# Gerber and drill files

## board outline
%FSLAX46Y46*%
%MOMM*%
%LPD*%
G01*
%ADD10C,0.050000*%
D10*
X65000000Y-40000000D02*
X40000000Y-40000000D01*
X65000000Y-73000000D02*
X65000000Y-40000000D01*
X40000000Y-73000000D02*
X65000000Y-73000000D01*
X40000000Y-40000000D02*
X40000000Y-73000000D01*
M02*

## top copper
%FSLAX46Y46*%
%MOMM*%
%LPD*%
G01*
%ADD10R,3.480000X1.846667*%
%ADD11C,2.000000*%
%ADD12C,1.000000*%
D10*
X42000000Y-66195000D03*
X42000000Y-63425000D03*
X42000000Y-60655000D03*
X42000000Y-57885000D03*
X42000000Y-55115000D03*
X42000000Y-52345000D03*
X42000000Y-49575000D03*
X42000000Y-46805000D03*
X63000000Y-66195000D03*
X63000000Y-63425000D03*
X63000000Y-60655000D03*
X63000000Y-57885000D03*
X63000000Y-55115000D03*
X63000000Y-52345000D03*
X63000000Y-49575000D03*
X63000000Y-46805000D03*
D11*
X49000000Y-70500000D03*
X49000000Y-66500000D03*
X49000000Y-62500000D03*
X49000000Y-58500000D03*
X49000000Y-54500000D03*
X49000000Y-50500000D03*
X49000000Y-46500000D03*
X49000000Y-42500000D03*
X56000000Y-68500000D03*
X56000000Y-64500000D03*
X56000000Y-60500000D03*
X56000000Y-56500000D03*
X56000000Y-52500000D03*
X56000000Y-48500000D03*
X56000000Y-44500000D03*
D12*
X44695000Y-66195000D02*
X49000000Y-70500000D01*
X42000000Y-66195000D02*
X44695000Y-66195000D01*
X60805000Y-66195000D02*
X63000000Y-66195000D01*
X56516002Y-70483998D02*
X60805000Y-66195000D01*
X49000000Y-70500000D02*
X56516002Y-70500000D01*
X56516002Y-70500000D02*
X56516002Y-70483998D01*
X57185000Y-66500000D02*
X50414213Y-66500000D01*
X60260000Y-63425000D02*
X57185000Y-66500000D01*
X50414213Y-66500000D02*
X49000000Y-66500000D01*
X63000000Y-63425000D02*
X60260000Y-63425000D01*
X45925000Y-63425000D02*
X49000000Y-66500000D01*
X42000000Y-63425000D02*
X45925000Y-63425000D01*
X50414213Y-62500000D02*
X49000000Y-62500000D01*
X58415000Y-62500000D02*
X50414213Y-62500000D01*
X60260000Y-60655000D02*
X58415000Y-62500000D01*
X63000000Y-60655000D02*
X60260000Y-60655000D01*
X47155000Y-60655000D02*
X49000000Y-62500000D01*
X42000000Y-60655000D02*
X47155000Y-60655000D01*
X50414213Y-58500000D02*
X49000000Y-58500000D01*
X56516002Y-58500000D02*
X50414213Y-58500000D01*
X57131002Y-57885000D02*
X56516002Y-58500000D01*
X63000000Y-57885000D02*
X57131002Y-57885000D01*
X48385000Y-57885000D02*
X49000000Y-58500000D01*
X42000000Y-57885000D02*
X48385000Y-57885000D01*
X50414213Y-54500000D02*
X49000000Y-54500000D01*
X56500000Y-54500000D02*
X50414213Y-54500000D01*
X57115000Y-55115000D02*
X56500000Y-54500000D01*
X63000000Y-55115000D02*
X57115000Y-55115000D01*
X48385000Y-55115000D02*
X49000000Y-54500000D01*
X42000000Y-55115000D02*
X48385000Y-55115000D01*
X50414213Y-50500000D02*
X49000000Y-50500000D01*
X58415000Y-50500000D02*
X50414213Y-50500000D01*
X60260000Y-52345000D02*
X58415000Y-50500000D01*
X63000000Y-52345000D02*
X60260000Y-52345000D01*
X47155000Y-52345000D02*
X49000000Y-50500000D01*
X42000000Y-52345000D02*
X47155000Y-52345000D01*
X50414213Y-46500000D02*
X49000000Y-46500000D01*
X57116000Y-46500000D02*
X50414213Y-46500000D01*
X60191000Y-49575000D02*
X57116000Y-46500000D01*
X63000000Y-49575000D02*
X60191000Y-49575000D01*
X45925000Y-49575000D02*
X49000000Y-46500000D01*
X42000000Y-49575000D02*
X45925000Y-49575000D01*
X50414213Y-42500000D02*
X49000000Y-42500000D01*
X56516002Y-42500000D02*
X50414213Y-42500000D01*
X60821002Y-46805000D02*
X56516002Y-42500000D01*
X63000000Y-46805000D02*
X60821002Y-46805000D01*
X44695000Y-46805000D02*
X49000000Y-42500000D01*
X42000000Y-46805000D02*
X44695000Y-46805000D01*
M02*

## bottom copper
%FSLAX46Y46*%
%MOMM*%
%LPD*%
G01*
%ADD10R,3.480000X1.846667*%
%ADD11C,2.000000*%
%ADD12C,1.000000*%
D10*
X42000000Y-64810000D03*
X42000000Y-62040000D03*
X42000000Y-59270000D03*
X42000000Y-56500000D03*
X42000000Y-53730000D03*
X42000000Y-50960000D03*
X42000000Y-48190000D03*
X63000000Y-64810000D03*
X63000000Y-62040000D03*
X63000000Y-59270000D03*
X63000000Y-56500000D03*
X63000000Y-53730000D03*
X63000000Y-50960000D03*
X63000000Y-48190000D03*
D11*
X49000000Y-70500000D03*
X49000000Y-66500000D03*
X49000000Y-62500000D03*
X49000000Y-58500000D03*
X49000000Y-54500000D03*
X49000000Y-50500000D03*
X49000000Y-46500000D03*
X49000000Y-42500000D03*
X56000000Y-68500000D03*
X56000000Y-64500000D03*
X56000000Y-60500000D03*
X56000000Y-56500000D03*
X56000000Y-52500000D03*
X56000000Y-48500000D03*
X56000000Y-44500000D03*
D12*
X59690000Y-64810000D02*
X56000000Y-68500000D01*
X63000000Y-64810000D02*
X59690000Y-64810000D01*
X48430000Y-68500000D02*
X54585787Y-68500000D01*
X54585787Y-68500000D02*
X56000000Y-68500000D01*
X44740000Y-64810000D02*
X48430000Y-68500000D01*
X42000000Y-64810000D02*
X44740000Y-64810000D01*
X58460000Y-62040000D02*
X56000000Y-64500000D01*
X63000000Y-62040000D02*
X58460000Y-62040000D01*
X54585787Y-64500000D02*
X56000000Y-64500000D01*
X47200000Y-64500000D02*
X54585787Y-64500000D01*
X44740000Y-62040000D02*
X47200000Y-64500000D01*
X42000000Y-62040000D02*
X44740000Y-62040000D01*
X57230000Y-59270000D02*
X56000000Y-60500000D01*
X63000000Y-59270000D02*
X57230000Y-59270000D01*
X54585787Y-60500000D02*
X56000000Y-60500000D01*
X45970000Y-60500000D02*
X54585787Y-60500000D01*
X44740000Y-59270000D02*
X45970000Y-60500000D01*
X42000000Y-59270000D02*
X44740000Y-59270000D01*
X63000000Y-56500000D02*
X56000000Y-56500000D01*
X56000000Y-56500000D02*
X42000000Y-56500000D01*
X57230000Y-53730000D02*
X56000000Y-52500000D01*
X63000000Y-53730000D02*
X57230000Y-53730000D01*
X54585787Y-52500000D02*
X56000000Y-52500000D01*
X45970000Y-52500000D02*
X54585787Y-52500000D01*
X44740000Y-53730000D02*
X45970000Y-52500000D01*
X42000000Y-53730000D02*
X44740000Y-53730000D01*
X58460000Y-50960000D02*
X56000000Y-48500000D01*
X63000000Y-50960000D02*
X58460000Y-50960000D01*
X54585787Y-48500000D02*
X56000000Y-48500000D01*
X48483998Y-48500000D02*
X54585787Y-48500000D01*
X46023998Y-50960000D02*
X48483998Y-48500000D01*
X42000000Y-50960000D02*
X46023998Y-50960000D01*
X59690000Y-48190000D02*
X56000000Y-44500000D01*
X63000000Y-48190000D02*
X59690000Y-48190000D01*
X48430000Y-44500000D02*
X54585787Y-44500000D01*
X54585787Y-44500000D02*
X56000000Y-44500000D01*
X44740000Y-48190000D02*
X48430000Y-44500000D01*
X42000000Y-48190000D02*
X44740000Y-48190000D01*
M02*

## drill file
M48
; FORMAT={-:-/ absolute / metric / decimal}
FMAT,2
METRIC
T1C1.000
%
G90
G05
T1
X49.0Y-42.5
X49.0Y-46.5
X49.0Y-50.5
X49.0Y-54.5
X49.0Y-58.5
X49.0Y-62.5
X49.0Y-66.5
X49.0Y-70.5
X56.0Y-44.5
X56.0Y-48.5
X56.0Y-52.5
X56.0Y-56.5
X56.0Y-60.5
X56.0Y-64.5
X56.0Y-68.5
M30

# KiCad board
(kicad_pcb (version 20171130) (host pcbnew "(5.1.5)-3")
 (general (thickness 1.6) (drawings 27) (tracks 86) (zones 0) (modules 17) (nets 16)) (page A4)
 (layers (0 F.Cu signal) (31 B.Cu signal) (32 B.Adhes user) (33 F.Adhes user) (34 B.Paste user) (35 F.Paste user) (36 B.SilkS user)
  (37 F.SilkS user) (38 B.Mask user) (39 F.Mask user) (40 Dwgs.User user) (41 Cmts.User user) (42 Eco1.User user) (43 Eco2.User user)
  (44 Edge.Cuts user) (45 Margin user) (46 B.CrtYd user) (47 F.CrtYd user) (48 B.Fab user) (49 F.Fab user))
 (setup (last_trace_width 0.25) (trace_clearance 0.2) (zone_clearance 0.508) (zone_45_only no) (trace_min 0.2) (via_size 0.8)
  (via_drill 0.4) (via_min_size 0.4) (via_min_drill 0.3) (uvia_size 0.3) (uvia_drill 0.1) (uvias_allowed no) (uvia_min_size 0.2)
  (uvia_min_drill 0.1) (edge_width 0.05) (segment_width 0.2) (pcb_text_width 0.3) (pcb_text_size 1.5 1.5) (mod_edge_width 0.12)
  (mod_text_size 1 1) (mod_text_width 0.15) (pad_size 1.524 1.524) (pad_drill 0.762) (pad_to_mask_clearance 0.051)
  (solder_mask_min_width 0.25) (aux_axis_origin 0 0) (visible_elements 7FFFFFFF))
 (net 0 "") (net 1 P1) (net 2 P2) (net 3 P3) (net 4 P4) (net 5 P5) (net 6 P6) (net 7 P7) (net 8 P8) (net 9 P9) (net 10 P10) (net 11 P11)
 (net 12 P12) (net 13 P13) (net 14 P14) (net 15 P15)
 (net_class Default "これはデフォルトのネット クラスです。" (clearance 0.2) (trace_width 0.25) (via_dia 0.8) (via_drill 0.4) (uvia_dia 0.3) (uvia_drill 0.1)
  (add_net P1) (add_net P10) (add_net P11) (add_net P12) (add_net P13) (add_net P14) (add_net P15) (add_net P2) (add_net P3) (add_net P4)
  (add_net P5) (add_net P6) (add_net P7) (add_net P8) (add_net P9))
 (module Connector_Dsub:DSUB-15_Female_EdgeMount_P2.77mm (layer F.Cu) (at 42 56.5 270)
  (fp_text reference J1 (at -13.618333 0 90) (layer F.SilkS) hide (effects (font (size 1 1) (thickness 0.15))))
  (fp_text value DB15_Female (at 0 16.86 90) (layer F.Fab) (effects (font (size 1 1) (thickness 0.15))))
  (pad 1 smd rect (at 9.695 0 270) (size 1.846667 3.48) (layers F.Cu F.Paste F.Mask) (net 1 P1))
  (pad 2 smd rect (at 6.925 0 270) (size 1.846667 3.48) (layers F.Cu F.Paste F.Mask) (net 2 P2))
  (pad 3 smd rect (at 4.155 0 270) (size 1.846667 3.48) (layers F.Cu F.Paste F.Mask) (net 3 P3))
  (pad 4 smd rect (at 1.385 0 270) (size 1.846667 3.48) (layers F.Cu F.Paste F.Mask) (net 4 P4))
  (pad 5 smd rect (at -1.385 0 270) (size 1.846667 3.48) (layers F.Cu F.Paste F.Mask) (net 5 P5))
  (pad 6 smd rect (at -4.155 0 270) (size 1.846667 3.48) (layers F.Cu F.Paste F.Mask) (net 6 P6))
  (pad 7 smd rect (at -6.925 0 270) (size 1.846667 3.48) (layers F.Cu F.Paste F.Mask) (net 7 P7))
  (pad 8 smd rect (at -9.695 0 270) (size 1.846667 3.48) (layers F.Cu F.Paste F.Mask) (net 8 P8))
  (pad 9 smd rect (at 8.31 0 270) (size 1.846667 3.48) (layers B.Cu B.Paste B.Mask) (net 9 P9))
  (pad 10 smd rect (at 5.54 0 270) (size 1.846667 3.48) (layers B.Cu B.Paste B.Mask) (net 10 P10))
  (pad 11 smd rect (at 2.77 0 270) (size 1.846667 3.48) (layers B.Cu B.Paste B.Mask) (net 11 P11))
  (pad 12 smd rect (at 0 0 270) (size 1.846667 3.48) (layers B.Cu B.Paste B.Mask) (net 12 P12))
  (pad 13 smd rect (at -2.77 0 270) (size 1.846667 3.48) (layers B.Cu B.Paste B.Mask) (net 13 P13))
  (pad 14 smd rect (at -5.54 0 270) (size 1.846667 3.48) (layers B.Cu B.Paste B.Mask) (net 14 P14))
  (pad 15 smd rect (at -8.31 0 270) (size 1.846667 3.48) (layers B.Cu B.Paste B.Mask) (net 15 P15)))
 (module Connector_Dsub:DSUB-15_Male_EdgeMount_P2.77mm (layer F.Cu) (at 63 56.5 90)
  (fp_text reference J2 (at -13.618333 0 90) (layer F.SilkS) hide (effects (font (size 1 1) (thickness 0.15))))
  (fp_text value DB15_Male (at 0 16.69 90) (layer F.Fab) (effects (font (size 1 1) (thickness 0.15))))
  (pad 1 smd rect (at -9.695 0 90) (size 1.846667 3.48) (layers F.Cu F.Paste F.Mask) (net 1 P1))
  (pad 2 smd rect (at -6.925 0 90) (size 1.846667 3.48) (layers F.Cu F.Paste F.Mask) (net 2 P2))
  (pad 3 smd rect (at -4.155 0 90) (size 1.846667 3.48) (layers F.Cu F.Paste F.Mask) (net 3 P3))
  (pad 4 smd rect (at -1.385 0 90) (size 1.846667 3.48) (layers F.Cu F.Paste F.Mask) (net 4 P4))
  (pad 5 smd rect (at 1.385 0 90) (size 1.846667 3.48) (layers F.Cu F.Paste F.Mask) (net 5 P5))
  (pad 6 smd rect (at 4.155 0 90) (size 1.846667 3.48) (layers F.Cu F.Paste F.Mask) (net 6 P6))
  (pad 7 smd rect (at 6.925 0 90) (size 1.846667 3.48) (layers F.Cu F.Paste F.Mask) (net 7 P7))
  (pad 8 smd rect (at 9.695 0 90) (size 1.846667 3.48) (layers F.Cu F.Paste F.Mask) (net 8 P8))
  (pad 9 smd rect (at -8.31 0 90) (size 1.846667 3.48) (layers B.Cu B.Paste B.Mask) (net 9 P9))
  (pad 10 smd rect (at -5.54 0 90) (size 1.846667 3.48) (layers B.Cu B.Paste B.Mask) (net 10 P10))
  (pad 11 smd rect (at -2.77 0 90) (size 1.846667 3.48) (layers B.Cu B.Paste B.Mask) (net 11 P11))
  (pad 12 smd rect (at 0 0 90) (size 1.846667 3.48) (layers B.Cu B.Paste B.Mask) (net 12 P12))
  (pad 13 smd rect (at 2.77 0 90) (size 1.846667 3.48) (layers B.Cu B.Paste B.Mask) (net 13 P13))
  (pad 14 smd rect (at 5.54 0 90) (size 1.846667 3.48) (layers B.Cu B.Paste B.Mask) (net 14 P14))
  (pad 15 smd rect (at 8.31 0 90) (size 1.846667 3.48) (layers B.Cu B.Paste B.Mask) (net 15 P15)))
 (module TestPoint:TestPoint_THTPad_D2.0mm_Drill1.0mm (layer F.Cu) (at 49 70.5)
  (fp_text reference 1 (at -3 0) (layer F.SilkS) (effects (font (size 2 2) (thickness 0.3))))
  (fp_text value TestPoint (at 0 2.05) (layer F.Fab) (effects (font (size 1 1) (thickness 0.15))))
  (pad 1 thru_hole circle (at 0 0) (size 2 2) (drill 1) (layers *.Cu *.Mask) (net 1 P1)))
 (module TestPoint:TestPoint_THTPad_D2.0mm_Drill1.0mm (layer F.Cu) (at 49 66.5)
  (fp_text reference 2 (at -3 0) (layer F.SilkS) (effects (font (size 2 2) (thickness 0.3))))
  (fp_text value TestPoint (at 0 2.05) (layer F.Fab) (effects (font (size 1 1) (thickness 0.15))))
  (pad 1 thru_hole circle (at 0 0) (size 2 2) (drill 1) (layers *.Cu *.Mask) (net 2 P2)))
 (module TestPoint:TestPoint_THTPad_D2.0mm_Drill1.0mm (layer F.Cu) (at 49 62.5)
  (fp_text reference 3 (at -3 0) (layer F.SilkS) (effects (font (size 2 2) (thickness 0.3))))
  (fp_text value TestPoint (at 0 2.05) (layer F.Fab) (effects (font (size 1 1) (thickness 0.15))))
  (pad 1 thru_hole circle (at 0 0) (size 2 2) (drill 1) (layers *.Cu *.Mask) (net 3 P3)))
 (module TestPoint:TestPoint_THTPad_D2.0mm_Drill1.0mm (layer F.Cu) (at 49 58.5)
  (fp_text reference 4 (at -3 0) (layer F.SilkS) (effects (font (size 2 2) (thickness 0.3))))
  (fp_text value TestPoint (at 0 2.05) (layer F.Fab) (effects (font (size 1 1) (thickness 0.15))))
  (pad 1 thru_hole circle (at 0 0) (size 2 2) (drill 1) (layers *.Cu *.Mask) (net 4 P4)))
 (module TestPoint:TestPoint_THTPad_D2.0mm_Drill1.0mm (layer F.Cu) (at 49 54.5)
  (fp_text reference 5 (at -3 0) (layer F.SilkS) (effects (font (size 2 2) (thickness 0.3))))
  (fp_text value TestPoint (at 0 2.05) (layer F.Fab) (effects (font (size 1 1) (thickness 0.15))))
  (pad 1 thru_hole circle (at 0 0) (size 2 2) (drill 1) (layers *.Cu *.Mask) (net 5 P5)))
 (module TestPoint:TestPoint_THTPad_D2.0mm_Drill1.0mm (layer F.Cu) (at 49 50.5)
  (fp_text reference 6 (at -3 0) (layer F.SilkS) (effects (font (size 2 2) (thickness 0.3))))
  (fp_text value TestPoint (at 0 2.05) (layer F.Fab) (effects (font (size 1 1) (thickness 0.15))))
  (pad 1 thru_hole circle (at 0 0) (size 2 2) (drill 1) (layers *.Cu *.Mask) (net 6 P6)))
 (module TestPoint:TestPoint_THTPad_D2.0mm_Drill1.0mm (layer F.Cu) (at 49 46.5)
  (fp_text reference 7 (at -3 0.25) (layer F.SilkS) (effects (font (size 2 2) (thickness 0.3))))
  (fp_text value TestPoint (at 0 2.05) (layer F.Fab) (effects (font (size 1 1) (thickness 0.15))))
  (pad 1 thru_hole circle (at 0 0) (size 2 2) (drill 1) (layers *.Cu *.Mask) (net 7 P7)))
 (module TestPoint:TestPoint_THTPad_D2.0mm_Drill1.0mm (layer F.Cu) (at 49 42.5)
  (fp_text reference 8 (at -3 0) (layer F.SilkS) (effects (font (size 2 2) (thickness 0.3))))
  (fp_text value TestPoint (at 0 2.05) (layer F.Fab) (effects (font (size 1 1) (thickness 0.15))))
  (pad 1 thru_hole circle (at 0 0) (size 2 2) (drill 1) (layers *.Cu *.Mask) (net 8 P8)))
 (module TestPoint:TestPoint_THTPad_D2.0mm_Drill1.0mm (layer F.Cu) (at 56 68.5)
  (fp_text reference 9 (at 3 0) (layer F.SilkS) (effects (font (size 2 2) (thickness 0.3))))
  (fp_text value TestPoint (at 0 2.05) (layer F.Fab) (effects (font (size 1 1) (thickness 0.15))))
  (pad 1 thru_hole circle (at 0 0) (size 2 2) (drill 1) (layers *.Cu *.Mask) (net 9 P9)))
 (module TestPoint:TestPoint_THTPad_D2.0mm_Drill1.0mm (layer F.Cu) (at 56 64.5)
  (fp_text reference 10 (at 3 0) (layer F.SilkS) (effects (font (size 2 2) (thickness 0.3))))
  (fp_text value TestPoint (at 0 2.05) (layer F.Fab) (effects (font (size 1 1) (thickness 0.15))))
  (pad 1 thru_hole circle (at 0 0) (size 2 2) (drill 1) (layers *.Cu *.Mask) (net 10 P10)))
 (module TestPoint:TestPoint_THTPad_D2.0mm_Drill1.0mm (layer F.Cu) (at 56 60.5)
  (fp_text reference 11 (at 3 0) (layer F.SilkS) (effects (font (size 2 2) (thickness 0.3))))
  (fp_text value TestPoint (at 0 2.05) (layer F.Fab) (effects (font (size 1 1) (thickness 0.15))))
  (pad 1 thru_hole circle (at 0 0) (size 2 2) (drill 1) (layers *.Cu *.Mask) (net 11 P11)))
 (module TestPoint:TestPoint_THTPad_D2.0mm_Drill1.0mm (layer F.Cu) (at 56 56.5)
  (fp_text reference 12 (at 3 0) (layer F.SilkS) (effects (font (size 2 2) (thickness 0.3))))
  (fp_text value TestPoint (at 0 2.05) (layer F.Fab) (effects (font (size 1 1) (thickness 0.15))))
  (pad 1 thru_hole circle (at 0 0) (size 2 2) (drill 1) (layers *.Cu *.Mask) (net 12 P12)))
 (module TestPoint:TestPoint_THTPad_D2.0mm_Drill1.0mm (layer F.Cu) (at 56 52.5)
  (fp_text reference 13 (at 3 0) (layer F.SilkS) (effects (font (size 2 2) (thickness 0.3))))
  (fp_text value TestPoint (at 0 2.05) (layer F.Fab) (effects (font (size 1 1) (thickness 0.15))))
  (pad 1 thru_hole circle (at 0 0) (size 2 2) (drill 1) (layers *.Cu *.Mask) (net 13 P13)))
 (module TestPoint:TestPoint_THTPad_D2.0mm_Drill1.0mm (layer F.Cu) (at 56 48.5)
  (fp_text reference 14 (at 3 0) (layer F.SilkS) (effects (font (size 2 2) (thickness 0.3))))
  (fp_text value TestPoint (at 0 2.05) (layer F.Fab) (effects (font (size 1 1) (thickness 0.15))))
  (pad 1 thru_hole circle (at 0 0) (size 2 2) (drill 1) (layers *.Cu *.Mask) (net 14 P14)))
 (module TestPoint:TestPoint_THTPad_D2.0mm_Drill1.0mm (layer F.Cu) (at 56 44.5)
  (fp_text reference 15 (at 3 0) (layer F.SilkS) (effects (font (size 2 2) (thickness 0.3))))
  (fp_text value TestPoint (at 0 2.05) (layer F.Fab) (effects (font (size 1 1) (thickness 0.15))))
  (pad 1 thru_hole circle (at 0 0) (size 2 2) (drill 1) (layers *.Cu *.Mask) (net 15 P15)))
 (gr_line (start 65 40) (end 40 40) (layer Edge.Cuts) (width 0.05))
 (gr_line (start 65 73) (end 65 40) (layer Edge.Cuts) (width 0.05))
 (gr_line (start 40 73) (end 65 73) (layer Edge.Cuts) (width 0.05))
 (gr_line (start 40 40) (end 40 73) (layer Edge.Cuts) (width 0.05))
 (segment (start 44.695 66.195) (end 49 70.5) (width 1) (layer F.Cu) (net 1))
 (segment (start 42 66.195) (end 44.695 66.195) (width 1) (layer F.Cu) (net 1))
 (segment (start 60.805 66.195) (end 63 66.195) (width 1) (layer F.Cu) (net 1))
 (segment (start 56.516002 70.483998) (end 60.805 66.195) (width 1) (layer F.Cu) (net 1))
 (segment (start 49 70.5) (end 56.516002 70.5) (width 1) (layer F.Cu) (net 1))
 (segment (start 56.516002 70.5) (end 56.516002 70.483998) (width 1) (layer F.Cu) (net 1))
 (segment (start 57.185 66.5) (end 50.414213 66.5) (width 1) (layer F.Cu) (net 2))
 (segment (start 60.26 63.425) (end 57.185 66.5) (width 1) (layer F.Cu) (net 2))
 (segment (start 50.414213 66.5) (end 49 66.5) (width 1) (layer F.Cu) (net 2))
 (segment (start 63 63.425) (end 60.26 63.425) (width 1) (layer F.Cu) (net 2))
 (segment (start 45.925 63.425) (end 49 66.5) (width 1) (layer F.Cu) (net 2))
 (segment (start 42 63.425) (end 45.925 63.425) (width 1) (layer F.Cu) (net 2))
 (segment (start 50.414213 62.5) (end 49 62.5) (width 1) (layer F.Cu) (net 3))
 (segment (start 58.415 62.5) (end 50.414213 62.5) (width 1) (layer F.Cu) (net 3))
 (segment (start 60.26 60.655) (end 58.415 62.5) (width 1) (layer F.Cu) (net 3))
 (segment (start 63 60.655) (end 60.26 60.655) (width 1) (layer F.Cu) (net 3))
 (segment (start 47.155 60.655) (end 49 62.5) (width 1) (layer F.Cu) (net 3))
 (segment (start 42 60.655) (end 47.155 60.655) (width 1) (layer F.Cu) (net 3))
 (segment (start 50.414213 58.5) (end 49 58.5) (width 1) (layer F.Cu) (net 4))
 (segment (start 56.516002 58.5) (end 50.414213 58.5) (width 1) (layer F.Cu) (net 4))
 (segment (start 57.131002 57.885) (end 56.516002 58.5) (width 1) (layer F.Cu) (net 4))
 (segment (start 63 57.885) (end 57.131002 57.885) (width 1) (layer F.Cu) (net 4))
 (segment (start 48.385 57.885) (end 49 58.5) (width 1) (layer F.Cu) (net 4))
 (segment (start 42 57.885) (end 48.385 57.885) (width 1) (layer F.Cu) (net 4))
 (segment (start 50.414213 54.5) (end 49 54.5) (width 1) (layer F.Cu) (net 5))
 (segment (start 56.5 54.5) (end 50.414213 54.5) (width 1) (layer F.Cu) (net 5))
 (segment (start 57.115 55.115) (end 56.5 54.5) (width 1) (layer F.Cu) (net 5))
 (segment (start 63 55.115) (end 57.115 55.115) (width 1) (layer F.Cu) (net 5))
 (segment (start 48.385 55.115) (end 49 54.5) (width 1) (layer F.Cu) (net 5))
 (segment (start 42 55.115) (end 48.385 55.115) (width 1) (layer F.Cu) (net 5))
 (segment (start 50.414213 50.5) (end 49 50.5) (width 1) (layer F.Cu) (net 6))
 (segment (start 58.415 50.5) (end 50.414213 50.5) (width 1) (layer F.Cu) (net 6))
 (segment (start 60.26 52.345) (end 58.415 50.5) (width 1) (layer F.Cu) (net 6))
 (segment (start 63 52.345) (end 60.26 52.345) (width 1) (layer F.Cu) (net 6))
 (segment (start 47.155 52.345) (end 49 50.5) (width 1) (layer F.Cu) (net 6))
 (segment (start 42 52.345) (end 47.155 52.345) (width 1) (layer F.Cu) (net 6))
 (segment (start 50.414213 46.5) (end 49 46.5) (width 1) (layer F.Cu) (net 7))
 (segment (start 57.116 46.5) (end 50.414213 46.5) (width 1) (layer F.Cu) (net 7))
 (segment (start 60.191 49.575) (end 57.116 46.5) (width 1) (layer F.Cu) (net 7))
 (segment (start 63 49.575) (end 60.191 49.575) (width 1) (layer F.Cu) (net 7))
 (segment (start 45.925 49.575) (end 49 46.5) (width 1) (layer F.Cu) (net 7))
 (segment (start 42 49.575) (end 45.925 49.575) (width 1) (layer F.Cu) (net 7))
 (segment (start 50.414213 42.5) (end 49 42.5) (width 1) (layer F.Cu) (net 8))
 (segment (start 56.516002 42.5) (end 50.414213 42.5) (width 1) (layer F.Cu) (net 8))
 (segment (start 60.821002 46.805) (end 56.516002 42.5) (width 1) (layer F.Cu) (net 8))
 (segment (start 63 46.805) (end 60.821002 46.805) (width 1) (layer F.Cu) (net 8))
 (segment (start 44.695 46.805) (end 49 42.5) (width 1) (layer F.Cu) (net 8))
 (segment (start 42 46.805) (end 44.695 46.805) (width 1) (layer F.Cu) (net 8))
 (segment (start 59.69 64.81) (end 56 68.5) (width 1) (layer B.Cu) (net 9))
 (segment (start 63 64.81) (end 59.69 64.81) (width 1) (layer B.Cu) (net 9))
 (segment (start 48.43 68.5) (end 54.585787 68.5) (width 1) (layer B.Cu) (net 9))
 (segment (start 54.585787 68.5) (end 56 68.5) (width 1) (layer B.Cu) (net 9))
 (segment (start 44.74 64.81) (end 48.43 68.5) (width 1) (layer B.Cu) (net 9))
 (segment (start 42 64.81) (end 44.74 64.81) (width 1) (layer B.Cu) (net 9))
 (segment (start 58.46 62.04) (end 56 64.5) (width 1) (layer B.Cu) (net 10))
 (segment (start 63 62.04) (end 58.46 62.04) (width 1) (layer B.Cu) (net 10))
 (segment (start 54.585787 64.5) (end 56 64.5) (width 1) (layer B.Cu) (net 10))
 (segment (start 47.2 64.5) (end 54.585787 64.5) (width 1) (layer B.Cu) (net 10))
 (segment (start 44.74 62.04) (end 47.2 64.5) (width 1) (layer B.Cu) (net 10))
 (segment (start 42 62.04) (end 44.74 62.04) (width 1) (layer B.Cu) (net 10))
 (segment (start 57.23 59.27) (end 56 60.5) (width 1) (layer B.Cu) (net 11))
 (segment (start 63 59.27) (end 57.23 59.27) (width 1) (layer B.Cu) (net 11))
 (segment (start 54.585787 60.5) (end 56 60.5) (width 1) (layer B.Cu) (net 11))
 (segment (start 45.97 60.5) (end 54.585787 60.5) (width 1) (layer B.Cu) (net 11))
 (segment (start 44.74 59.27) (end 45.97 60.5) (width 1) (layer B.Cu) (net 11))
 (segment (start 42 59.27) (end 44.74 59.27) (width 1) (layer B.Cu) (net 11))
 (segment (start 63 56.5) (end 56 56.5) (width 1) (layer B.Cu) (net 12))
 (segment (start 56 56.5) (end 42 56.5) (width 1) (layer B.Cu) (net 12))
 (segment (start 57.23 53.73) (end 56 52.5) (width 1) (layer B.Cu) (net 13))
 (segment (start 63 53.73) (end 57.23 53.73) (width 1) (layer B.Cu) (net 13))
 (segment (start 54.585787 52.5) (end 56 52.5) (width 1) (layer B.Cu) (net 13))
 (segment (start 45.97 52.5) (end 54.585787 52.5) (width 1) (layer B.Cu) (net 13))
 (segment (start 44.74 53.73) (end 45.97 52.5) (width 1) (layer B.Cu) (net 13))
 (segment (start 42 53.73) (end 44.74 53.73) (width 1) (layer B.Cu) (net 13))
 (segment (start 58.46 50.96) (end 56 48.5) (width 1) (layer B.Cu) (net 14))
 (segment (start 63 50.96) (end 58.46 50.96) (width 1) (layer B.Cu) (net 14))
 (segment (start 54.585787 48.5) (end 56 48.5) (width 1) (layer B.Cu) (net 14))
 (segment (start 48.483998 48.5) (end 54.585787 48.5) (width 1) (layer B.Cu) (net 14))
 (segment (start 46.023998 50.96) (end 48.483998 48.5) (width 1) (layer B.Cu) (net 14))
 (segment (start 42 50.96) (end 46.023998 50.96) (width 1) (layer B.Cu) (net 14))
 (segment (start 59.69 48.19) (end 56 44.5) (width 1) (layer B.Cu) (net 15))
 (segment (start 63 48.19) (end 59.69 48.19) (width 1) (layer B.Cu) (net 15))
 (segment (start 48.43 44.5) (end 54.585787 44.5) (width 1) (layer B.Cu) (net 15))
 (segment (start 54.585787 44.5) (end 56 44.5) (width 1) (layer B.Cu) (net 15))
 (segment (start 44.74 48.19) (end 48.43 44.5) (width 1) (layer B.Cu) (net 15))
 (segment (start 42 48.19) (end 44.74 48.19) (width 1) (layer B.Cu) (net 15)))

